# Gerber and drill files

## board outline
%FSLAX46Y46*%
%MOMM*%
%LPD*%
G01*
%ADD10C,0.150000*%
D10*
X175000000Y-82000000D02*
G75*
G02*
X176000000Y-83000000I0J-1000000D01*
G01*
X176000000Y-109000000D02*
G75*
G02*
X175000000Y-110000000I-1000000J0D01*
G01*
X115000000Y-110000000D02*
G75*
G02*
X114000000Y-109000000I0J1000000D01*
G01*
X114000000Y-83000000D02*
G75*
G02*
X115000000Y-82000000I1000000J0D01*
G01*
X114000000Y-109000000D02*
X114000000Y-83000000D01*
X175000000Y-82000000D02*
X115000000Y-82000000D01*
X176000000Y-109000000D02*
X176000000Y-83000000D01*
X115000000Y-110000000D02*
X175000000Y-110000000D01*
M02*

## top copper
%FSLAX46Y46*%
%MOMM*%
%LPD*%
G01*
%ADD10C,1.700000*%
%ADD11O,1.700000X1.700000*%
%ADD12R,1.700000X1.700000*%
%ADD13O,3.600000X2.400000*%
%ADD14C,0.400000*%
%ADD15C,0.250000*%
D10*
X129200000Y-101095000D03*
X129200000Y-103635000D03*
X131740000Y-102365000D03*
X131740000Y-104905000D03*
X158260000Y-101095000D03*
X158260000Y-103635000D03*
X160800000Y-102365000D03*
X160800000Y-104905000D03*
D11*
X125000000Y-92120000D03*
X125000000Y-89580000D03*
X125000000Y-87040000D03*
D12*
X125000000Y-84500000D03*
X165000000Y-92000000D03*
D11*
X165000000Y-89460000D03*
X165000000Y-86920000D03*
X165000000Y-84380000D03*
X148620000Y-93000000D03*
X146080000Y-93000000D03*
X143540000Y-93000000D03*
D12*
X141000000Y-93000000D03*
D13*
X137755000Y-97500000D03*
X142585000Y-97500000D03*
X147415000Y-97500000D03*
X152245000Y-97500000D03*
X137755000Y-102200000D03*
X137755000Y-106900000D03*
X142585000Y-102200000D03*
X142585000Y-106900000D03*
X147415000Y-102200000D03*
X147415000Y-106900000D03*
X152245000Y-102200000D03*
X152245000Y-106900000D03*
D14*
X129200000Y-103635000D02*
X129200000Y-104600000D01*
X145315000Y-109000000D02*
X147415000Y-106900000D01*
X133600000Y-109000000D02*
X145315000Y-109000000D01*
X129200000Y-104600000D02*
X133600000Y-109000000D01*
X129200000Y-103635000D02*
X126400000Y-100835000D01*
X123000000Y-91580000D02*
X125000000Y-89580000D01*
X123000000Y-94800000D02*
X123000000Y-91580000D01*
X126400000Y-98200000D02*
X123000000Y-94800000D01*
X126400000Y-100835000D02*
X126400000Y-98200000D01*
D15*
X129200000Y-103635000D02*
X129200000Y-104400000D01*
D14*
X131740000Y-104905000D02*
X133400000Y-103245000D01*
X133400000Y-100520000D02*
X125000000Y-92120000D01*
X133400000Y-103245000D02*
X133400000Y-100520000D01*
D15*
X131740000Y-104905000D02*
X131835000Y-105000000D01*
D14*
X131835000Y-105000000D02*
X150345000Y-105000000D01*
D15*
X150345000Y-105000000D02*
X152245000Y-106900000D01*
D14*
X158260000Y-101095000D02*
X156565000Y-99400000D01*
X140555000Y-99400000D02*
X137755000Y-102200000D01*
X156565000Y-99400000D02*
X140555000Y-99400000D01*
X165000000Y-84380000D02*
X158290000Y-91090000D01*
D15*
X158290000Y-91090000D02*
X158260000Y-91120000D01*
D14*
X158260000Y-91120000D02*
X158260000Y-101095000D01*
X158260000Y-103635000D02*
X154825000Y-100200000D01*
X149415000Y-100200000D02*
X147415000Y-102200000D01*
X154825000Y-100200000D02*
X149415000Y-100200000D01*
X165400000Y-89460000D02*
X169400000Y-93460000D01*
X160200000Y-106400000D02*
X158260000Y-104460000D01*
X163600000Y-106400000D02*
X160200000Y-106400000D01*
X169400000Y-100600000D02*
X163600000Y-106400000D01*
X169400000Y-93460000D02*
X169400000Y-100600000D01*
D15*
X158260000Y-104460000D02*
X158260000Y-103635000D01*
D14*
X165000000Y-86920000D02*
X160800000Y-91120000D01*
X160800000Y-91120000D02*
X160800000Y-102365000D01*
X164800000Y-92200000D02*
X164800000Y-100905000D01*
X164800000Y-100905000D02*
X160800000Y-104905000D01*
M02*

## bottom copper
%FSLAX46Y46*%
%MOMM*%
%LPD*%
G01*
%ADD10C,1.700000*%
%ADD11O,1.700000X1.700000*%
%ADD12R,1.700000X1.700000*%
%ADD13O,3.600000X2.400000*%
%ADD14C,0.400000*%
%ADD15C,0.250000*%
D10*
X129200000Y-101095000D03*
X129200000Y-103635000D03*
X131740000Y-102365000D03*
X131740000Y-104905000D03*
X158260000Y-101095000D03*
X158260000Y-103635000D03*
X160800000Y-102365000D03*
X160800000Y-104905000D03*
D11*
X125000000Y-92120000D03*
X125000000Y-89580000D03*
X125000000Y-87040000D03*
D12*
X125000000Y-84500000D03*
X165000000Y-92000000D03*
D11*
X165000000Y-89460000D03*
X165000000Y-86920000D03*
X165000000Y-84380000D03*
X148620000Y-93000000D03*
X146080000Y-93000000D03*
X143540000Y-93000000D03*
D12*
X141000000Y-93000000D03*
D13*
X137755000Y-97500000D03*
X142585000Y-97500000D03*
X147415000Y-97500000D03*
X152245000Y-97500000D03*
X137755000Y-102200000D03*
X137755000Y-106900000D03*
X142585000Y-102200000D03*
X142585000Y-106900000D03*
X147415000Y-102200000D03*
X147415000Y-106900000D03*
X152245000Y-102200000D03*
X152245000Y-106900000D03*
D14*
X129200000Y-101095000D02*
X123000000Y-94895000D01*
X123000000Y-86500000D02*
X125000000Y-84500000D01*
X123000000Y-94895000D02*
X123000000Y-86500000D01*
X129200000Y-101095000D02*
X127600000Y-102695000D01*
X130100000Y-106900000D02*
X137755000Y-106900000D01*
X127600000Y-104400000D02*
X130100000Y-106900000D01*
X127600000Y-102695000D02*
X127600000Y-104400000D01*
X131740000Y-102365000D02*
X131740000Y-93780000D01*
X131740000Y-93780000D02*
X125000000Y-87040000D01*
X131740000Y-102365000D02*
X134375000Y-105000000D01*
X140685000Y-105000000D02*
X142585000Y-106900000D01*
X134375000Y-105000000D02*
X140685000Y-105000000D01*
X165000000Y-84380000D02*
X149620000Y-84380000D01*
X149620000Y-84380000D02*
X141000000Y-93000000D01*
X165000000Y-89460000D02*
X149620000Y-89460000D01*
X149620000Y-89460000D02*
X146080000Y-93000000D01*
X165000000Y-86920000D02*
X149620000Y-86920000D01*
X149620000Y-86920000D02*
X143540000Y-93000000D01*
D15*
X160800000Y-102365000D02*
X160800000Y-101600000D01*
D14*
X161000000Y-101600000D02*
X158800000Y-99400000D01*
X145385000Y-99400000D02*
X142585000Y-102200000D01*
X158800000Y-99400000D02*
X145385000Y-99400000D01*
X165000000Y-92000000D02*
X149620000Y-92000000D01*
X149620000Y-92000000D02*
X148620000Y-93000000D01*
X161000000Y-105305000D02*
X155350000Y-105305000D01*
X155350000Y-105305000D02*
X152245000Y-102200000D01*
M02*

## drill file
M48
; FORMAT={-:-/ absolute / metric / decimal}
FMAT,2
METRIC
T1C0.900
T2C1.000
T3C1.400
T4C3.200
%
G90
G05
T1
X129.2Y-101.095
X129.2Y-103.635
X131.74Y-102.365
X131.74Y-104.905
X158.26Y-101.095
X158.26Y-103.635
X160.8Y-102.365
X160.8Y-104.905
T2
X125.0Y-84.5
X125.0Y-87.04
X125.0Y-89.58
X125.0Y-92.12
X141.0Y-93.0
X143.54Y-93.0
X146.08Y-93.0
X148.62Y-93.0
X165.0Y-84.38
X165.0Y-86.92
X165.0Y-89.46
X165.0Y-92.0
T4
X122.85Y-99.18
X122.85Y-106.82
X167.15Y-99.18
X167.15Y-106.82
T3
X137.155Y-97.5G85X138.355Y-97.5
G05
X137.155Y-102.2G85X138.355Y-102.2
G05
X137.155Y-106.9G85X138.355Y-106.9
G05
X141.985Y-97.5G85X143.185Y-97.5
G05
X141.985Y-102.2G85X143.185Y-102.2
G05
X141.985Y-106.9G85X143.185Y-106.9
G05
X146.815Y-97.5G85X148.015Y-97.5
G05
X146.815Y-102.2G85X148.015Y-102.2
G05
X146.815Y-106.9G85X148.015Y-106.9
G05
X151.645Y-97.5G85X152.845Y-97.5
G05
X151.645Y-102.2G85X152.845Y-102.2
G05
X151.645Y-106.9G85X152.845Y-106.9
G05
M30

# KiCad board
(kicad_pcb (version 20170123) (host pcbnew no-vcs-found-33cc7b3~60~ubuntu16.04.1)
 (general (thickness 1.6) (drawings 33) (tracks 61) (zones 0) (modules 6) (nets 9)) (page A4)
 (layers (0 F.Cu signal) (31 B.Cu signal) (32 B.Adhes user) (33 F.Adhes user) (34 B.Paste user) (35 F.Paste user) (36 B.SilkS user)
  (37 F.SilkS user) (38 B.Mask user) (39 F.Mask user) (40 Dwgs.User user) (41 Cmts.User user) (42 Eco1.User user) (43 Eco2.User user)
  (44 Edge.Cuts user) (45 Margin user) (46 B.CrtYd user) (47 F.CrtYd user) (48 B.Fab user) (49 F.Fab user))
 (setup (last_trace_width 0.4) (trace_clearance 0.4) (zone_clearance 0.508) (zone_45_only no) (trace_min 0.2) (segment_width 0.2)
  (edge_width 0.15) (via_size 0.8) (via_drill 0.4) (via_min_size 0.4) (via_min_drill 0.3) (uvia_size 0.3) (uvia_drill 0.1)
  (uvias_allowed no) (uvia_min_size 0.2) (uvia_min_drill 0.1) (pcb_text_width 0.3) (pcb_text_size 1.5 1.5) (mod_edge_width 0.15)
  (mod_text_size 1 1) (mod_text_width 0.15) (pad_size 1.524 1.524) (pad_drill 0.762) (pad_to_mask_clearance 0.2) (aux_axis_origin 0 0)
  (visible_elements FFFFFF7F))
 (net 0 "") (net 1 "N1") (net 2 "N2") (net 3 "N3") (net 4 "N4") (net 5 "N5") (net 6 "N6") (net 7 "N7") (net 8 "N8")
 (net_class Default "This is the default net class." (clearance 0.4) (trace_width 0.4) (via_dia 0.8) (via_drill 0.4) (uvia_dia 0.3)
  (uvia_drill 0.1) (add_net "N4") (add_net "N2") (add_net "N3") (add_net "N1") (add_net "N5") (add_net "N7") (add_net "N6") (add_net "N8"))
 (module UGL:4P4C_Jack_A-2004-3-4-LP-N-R (layer F.Cu) (at 115 103 270)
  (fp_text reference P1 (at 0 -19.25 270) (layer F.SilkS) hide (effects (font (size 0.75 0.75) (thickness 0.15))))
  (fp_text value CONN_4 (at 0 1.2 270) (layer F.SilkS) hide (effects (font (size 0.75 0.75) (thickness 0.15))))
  (pad "" np_thru_hole circle (at -3.82 -7.85 270) (size 3.2 3.2) (drill 3.2) (layers *.Cu *.Mask F.SilkS))
  (pad "" np_thru_hole circle (at 3.82 -7.85 270) (size 3.2 3.2) (drill 3.2) (layers *.Cu *.Mask F.SilkS))
  (pad 4 thru_hole circle (at -1.905 -14.2 270) (size 1.7 1.7) (drill 0.9) (layers *.Cu *.Mask F.SilkS) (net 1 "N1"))
  (pad 2 thru_hole circle (at 0.635 -14.2 270) (size 1.7 1.7) (drill 0.9) (layers *.Cu *.Mask F.SilkS) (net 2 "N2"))
  (pad 3 thru_hole circle (at -0.635 -16.74 270) (size 1.7 1.7) (drill 0.9) (layers *.Cu *.Mask F.SilkS) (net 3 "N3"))
  (pad 1 thru_hole circle (at 1.905 -16.74 270) (size 1.7 1.7) (drill 0.9) (layers *.Cu *.Mask F.SilkS) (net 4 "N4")))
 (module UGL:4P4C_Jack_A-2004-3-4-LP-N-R (layer F.Cu) (at 175 103 90)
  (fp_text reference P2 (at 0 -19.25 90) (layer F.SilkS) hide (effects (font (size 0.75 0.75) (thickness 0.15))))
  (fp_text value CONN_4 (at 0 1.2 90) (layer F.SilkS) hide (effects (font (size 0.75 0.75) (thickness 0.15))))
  (pad 1 thru_hole circle (at 1.905 -16.74 90) (size 1.7 1.7) (drill 0.9) (layers *.Cu *.Mask F.SilkS) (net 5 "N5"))
  (pad 3 thru_hole circle (at -0.635 -16.74 90) (size 1.7 1.7) (drill 0.9) (layers *.Cu *.Mask F.SilkS) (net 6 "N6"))
  (pad 2 thru_hole circle (at 0.635 -14.2 90) (size 1.7 1.7) (drill 0.9) (layers *.Cu *.Mask F.SilkS) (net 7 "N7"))
  (pad 4 thru_hole circle (at -1.905 -14.2 90) (size 1.7 1.7) (drill 0.9) (layers *.Cu *.Mask F.SilkS) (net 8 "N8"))
  (pad "" np_thru_hole circle (at 3.82 -7.85 90) (size 3.2 3.2) (drill 3.2) (layers *.Cu *.Mask F.SilkS))
  (pad "" np_thru_hole circle (at -3.82 -7.85 90) (size 3.2 3.2) (drill 3.2) (layers *.Cu *.Mask F.SilkS)))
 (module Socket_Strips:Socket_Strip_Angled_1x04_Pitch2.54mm (layer F.Cu) (at 125 84.5)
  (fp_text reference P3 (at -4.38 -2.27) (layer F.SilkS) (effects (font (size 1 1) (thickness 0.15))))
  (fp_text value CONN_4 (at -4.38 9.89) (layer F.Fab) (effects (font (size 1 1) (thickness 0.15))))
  (pad 4 thru_hole oval (at 0 7.62) (size 1.7 1.7) (drill 1) (layers *.Cu *.Mask) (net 4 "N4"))
  (pad 3 thru_hole oval (at 0 5.08) (size 1.7 1.7) (drill 1) (layers *.Cu *.Mask) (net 2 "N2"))
  (pad 2 thru_hole oval (at 0 2.54) (size 1.7 1.7) (drill 1) (layers *.Cu *.Mask) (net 3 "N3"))
  (pad 1 thru_hole rect (at 0 0) (size 1.7 1.7) (drill 1) (layers *.Cu *.Mask) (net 1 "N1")))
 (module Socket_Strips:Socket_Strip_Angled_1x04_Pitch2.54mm (layer F.Cu) (at 165 92 180)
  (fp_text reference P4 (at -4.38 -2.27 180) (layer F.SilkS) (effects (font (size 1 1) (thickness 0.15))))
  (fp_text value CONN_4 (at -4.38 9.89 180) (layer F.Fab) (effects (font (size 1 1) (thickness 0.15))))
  (pad 1 thru_hole rect (at 0 0 180) (size 1.7 1.7) (drill 1) (layers *.Cu *.Mask) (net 8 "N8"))
  (pad 2 thru_hole oval (at 0 2.54 180) (size 1.7 1.7) (drill 1) (layers *.Cu *.Mask) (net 6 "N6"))
  (pad 3 thru_hole oval (at 0 5.08 180) (size 1.7 1.7) (drill 1) (layers *.Cu *.Mask) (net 7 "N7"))
  (pad 4 thru_hole oval (at 0 7.62 180) (size 1.7 1.7) (drill 1) (layers *.Cu *.Mask) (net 5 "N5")))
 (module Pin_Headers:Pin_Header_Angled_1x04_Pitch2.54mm (layer F.Cu) (at 141 93 90)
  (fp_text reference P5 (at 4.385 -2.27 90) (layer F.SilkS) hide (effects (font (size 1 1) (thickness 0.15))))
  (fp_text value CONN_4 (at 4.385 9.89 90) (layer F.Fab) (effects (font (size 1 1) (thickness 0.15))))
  (pad 4 thru_hole oval (at 0 7.62 90) (size 1.7 1.7) (drill 1) (layers *.Cu *.Mask) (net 8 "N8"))
  (pad 3 thru_hole oval (at 0 5.08 90) (size 1.7 1.7) (drill 1) (layers *.Cu *.Mask) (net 6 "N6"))
  (pad 2 thru_hole oval (at 0 2.54 90) (size 1.7 1.7) (drill 1) (layers *.Cu *.Mask) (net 7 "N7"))
  (pad 1 thru_hole rect (at 0 0 90) (size 1.7 1.7) (drill 1) (layers *.Cu *.Mask) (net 5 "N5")))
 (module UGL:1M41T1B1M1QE (layer F.Cu) (at 145 102.2)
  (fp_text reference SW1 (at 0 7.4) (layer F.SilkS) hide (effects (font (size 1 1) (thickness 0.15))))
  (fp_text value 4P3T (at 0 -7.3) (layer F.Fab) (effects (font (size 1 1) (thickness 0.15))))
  (pad "" thru_hole oval (at -7.245 -4.7) (size 3.6 2.4) (drill oval 2.6 1.4) (layers *.Cu *.Mask))
  (pad "" thru_hole oval (at -2.415 -4.7) (size 3.6 2.4) (drill oval 2.6 1.4) (layers *.Cu *.Mask))
  (pad "" thru_hole oval (at 2.415 -4.7) (size 3.6 2.4) (drill oval 2.6 1.4) (layers *.Cu *.Mask))
  (pad "" thru_hole oval (at 7.245 -4.7) (size 3.6 2.4) (drill oval 2.6 1.4) (layers *.Cu *.Mask))
  (pad 8 thru_hole oval (at -7.245 0) (size 3.6 2.4) (drill oval 2.6 1.4) (layers *.Cu *.Mask) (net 5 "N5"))
  (pad 7 thru_hole oval (at -7.245 4.7) (size 3.6 2.4) (drill oval 2.6 1.4) (layers *.Cu *.Mask) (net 1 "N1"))
  (pad 6 thru_hole oval (at -2.415 0) (size 3.6 2.4) (drill oval 2.6 1.4) (layers *.Cu *.Mask) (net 7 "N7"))
  (pad 5 thru_hole oval (at -2.415 4.7) (size 3.6 2.4) (drill oval 2.6 1.4) (layers *.Cu *.Mask) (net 3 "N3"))
  (pad 4 thru_hole oval (at 2.415 0) (size 3.6 2.4) (drill oval 2.6 1.4) (layers *.Cu *.Mask) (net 6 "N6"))
  (pad 3 thru_hole oval (at 2.415 4.7) (size 3.6 2.4) (drill oval 2.6 1.4) (layers *.Cu *.Mask) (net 2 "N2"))
  (pad 2 thru_hole oval (at 7.245 0) (size 3.6 2.4) (drill oval 2.6 1.4) (layers *.Cu *.Mask) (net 8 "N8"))
  (pad 1 thru_hole oval (at 7.245 4.7) (size 3.6 2.4) (drill oval 2.6 1.4) (layers *.Cu *.Mask) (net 4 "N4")))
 (gr_arc (start 175 83) (end 175 82) (angle 90) (layer Edge.Cuts) (width 0.15))
 (gr_arc (start 175 109) (end 176 109) (angle 90) (layer Edge.Cuts) (width 0.15))
 (gr_arc (start 115 109) (end 115 110) (angle 90) (layer Edge.Cuts) (width 0.15))
 (gr_arc (start 115 83) (end 114 83) (angle 90) (layer Edge.Cuts) (width 0.15))
 (gr_line (start 114 109) (end 114 83) (angle 90) (layer Edge.Cuts) (width 0.15))
 (gr_line (start 175 82) (end 115 82) (angle 90) (layer Edge.Cuts) (width 0.15))
 (gr_line (start 176 109) (end 176 83) (angle 90) (layer Edge.Cuts) (width 0.15))
 (gr_line (start 115 110) (end 175 110) (angle 90) (layer Edge.Cuts) (width 0.15))
 (segment (start 129.2 101.095) (end 123 94.895) (width 0.4) (layer B.Cu) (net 1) (status 400000))
 (segment (start 123 86.5) (end 125 84.5) (width 0.4) (layer B.Cu) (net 1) (status 800000))
 (segment (start 123 94.895) (end 123 86.5) (width 0.4) (layer B.Cu) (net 1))
 (segment (start 129.2 101.095) (end 127.6 102.695) (width 0.4) (layer B.Cu) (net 1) (status 400000))
 (segment (start 130.1 106.9) (end 137.755 106.9) (width 0.4) (layer B.Cu) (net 1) (status 800000))
 (segment (start 127.6 104.4) (end 130.1 106.9) (width 0.4) (layer B.Cu) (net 1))
 (segment (start 127.6 102.695) (end 127.6 104.4) (width 0.4) (layer B.Cu) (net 1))
 (segment (start 129.2 103.635) (end 129.2 104.6) (width 0.4) (layer F.Cu) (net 2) (status 400000))
 (segment (start 145.315 109) (end 147.415 106.9) (width 0.4) (layer F.Cu) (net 2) (status 800000))
 (segment (start 133.6 109) (end 145.315 109) (width 0.4) (layer F.Cu) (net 2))
 (segment (start 129.2 104.6) (end 133.6 109) (width 0.4) (layer F.Cu) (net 2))
 (segment (start 129.2 103.635) (end 126.4 100.835) (width 0.4) (layer F.Cu) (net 2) (status 400000))
 (segment (start 123 91.58) (end 125 89.58) (width 0.4) (layer F.Cu) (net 2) (status 800000))
 (segment (start 123 94.8) (end 123 91.58) (width 0.4) (layer F.Cu) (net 2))
 (segment (start 126.4 98.2) (end 123 94.8) (width 0.4) (layer F.Cu) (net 2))
 (segment (start 126.4 100.835) (end 126.4 98.2) (width 0.4) (layer F.Cu) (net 2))
 (segment (start 129.2 103.635) (end 129.2 104.4) (width 0.25) (layer F.Cu) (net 2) (status C00000))
 (segment (start 131.74 102.365) (end 131.74 93.78) (width 0.4) (layer B.Cu) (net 3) (status 400000))
 (segment (start 131.74 93.78) (end 125 87.04) (width 0.4) (layer B.Cu) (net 3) (status 800000))
 (segment (start 131.74 102.365) (end 134.375 105) (width 0.4) (layer B.Cu) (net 3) (status 400000))
 (segment (start 140.685 105) (end 142.585 106.9) (width 0.4) (layer B.Cu) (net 3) (status 800000))
 (segment (start 134.375 105) (end 140.685 105) (width 0.4) (layer B.Cu) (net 3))
 (segment (start 131.74 104.905) (end 133.4 103.245) (width 0.4) (layer F.Cu) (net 4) (status 400000))
 (segment (start 133.4 100.52) (end 125 92.12) (width 0.4) (layer F.Cu) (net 4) (status 800000))
 (segment (start 133.4 103.245) (end 133.4 100.52) (width 0.4) (layer F.Cu) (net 4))
 (segment (start 131.74 104.905) (end 131.835 105) (width 0.25) (layer F.Cu) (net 4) (status C00000))
 (segment (start 131.835 105) (end 150.345 105) (width 0.4) (layer F.Cu) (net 4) (status 400000))
 (segment (start 150.345 105) (end 152.245 106.9) (width 0.25) (layer F.Cu) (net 4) (status 800000))
 (segment (start 165 84.38) (end 149.62 84.38) (width 0.4) (layer B.Cu) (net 5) (status 400000))
 (segment (start 149.62 84.38) (end 141 93) (width 0.4) (layer B.Cu) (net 5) (status 800000))
 (segment (start 158.26 101.095) (end 156.565 99.4) (width 0.4) (layer F.Cu) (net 5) (status 400000))
 (segment (start 140.555 99.4) (end 137.755 102.2) (width 0.4) (layer F.Cu) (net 5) (status 800000))
 (segment (start 156.565 99.4) (end 140.555 99.4) (width 0.4) (layer F.Cu) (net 5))
 (segment (start 165 84.38) (end 158.29 91.09) (width 0.4) (layer F.Cu) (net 5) (status 400000))
 (segment (start 158.29 91.09) (end 158.26 91.12) (width 0.25) (layer F.Cu) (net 5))
 (segment (start 158.26 91.12) (end 158.26 101.095) (width 0.4) (layer F.Cu) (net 5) (status 800000))
 (segment (start 165 89.46) (end 149.62 89.46) (width 0.4) (layer B.Cu) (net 6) (status 400000))
 (segment (start 149.62 89.46) (end 146.08 93) (width 0.4) (layer B.Cu) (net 6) (status 800000))
 (segment (start 158.26 103.635) (end 154.825 100.2) (width 0.4) (layer F.Cu) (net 6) (status 400000))
 (segment (start 149.415 100.2) (end 147.415 102.2) (width 0.4) (layer F.Cu) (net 6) (status 800000))
 (segment (start 154.825 100.2) (end 149.415 100.2) (width 0.4) (layer F.Cu) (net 6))
 (segment (start 165.4 89.46) (end 169.4 93.46) (width 0.4) (layer F.Cu) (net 6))
 (segment (start 160.2 106.4) (end 158.26 104.46) (width 0.4) (layer F.Cu) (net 6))
 (segment (start 163.6 106.4) (end 160.2 106.4) (width 0.4) (layer F.Cu) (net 6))
 (segment (start 169.4 100.6) (end 163.6 106.4) (width 0.4) (layer F.Cu) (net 6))
 (segment (start 169.4 93.46) (end 169.4 100.6) (width 0.4) (layer F.Cu) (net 6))
 (segment (start 158.26 104.46) (end 158.26 103.635) (width 0.25) (layer F.Cu) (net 6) (status 800000))
 (segment (start 165 86.92) (end 149.62 86.92) (width 0.4) (layer B.Cu) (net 7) (status 400000))
 (segment (start 149.62 86.92) (end 143.54 93) (width 0.4) (layer B.Cu) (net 7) (status 800000))
 (segment (start 160.8 102.365) (end 160.8 101.6) (width 0.25) (layer B.Cu) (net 7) (status C00000))
 (segment (start 161 101.6) (end 158.8 99.4) (width 0.4) (layer B.Cu) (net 7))
 (segment (start 145.385 99.4) (end 142.585 102.2) (width 0.4) (layer B.Cu) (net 7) (status 800000))
 (segment (start 158.8 99.4) (end 145.385 99.4) (width 0.4) (layer B.Cu) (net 7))
 (segment (start 165 86.92) (end 160.8 91.12) (width 0.4) (layer F.Cu) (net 7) (status 400000))
 (segment (start 160.8 91.12) (end 160.8 102.365) (width 0.4) (layer F.Cu) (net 7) (status 800000))
 (segment (start 165 92) (end 149.62 92) (width 0.4) (layer B.Cu) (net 8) (status 400000))
 (segment (start 149.62 92) (end 148.62 93) (width 0.4) (layer B.Cu) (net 8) (status 800000))
 (segment (start 161 105.305) (end 155.35 105.305) (width 0.4) (layer B.Cu) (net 8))
 (segment (start 155.35 105.305) (end 152.245 102.2) (width 0.4) (layer B.Cu) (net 8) (status 800000))
 (segment (start 164.8 92.2) (end 164.8 100.905) (width 0.4) (layer F.Cu) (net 8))
 (segment (start 164.8 100.905) (end 160.8 104.905) (width 0.4) (layer F.Cu) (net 8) (status 800000)))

